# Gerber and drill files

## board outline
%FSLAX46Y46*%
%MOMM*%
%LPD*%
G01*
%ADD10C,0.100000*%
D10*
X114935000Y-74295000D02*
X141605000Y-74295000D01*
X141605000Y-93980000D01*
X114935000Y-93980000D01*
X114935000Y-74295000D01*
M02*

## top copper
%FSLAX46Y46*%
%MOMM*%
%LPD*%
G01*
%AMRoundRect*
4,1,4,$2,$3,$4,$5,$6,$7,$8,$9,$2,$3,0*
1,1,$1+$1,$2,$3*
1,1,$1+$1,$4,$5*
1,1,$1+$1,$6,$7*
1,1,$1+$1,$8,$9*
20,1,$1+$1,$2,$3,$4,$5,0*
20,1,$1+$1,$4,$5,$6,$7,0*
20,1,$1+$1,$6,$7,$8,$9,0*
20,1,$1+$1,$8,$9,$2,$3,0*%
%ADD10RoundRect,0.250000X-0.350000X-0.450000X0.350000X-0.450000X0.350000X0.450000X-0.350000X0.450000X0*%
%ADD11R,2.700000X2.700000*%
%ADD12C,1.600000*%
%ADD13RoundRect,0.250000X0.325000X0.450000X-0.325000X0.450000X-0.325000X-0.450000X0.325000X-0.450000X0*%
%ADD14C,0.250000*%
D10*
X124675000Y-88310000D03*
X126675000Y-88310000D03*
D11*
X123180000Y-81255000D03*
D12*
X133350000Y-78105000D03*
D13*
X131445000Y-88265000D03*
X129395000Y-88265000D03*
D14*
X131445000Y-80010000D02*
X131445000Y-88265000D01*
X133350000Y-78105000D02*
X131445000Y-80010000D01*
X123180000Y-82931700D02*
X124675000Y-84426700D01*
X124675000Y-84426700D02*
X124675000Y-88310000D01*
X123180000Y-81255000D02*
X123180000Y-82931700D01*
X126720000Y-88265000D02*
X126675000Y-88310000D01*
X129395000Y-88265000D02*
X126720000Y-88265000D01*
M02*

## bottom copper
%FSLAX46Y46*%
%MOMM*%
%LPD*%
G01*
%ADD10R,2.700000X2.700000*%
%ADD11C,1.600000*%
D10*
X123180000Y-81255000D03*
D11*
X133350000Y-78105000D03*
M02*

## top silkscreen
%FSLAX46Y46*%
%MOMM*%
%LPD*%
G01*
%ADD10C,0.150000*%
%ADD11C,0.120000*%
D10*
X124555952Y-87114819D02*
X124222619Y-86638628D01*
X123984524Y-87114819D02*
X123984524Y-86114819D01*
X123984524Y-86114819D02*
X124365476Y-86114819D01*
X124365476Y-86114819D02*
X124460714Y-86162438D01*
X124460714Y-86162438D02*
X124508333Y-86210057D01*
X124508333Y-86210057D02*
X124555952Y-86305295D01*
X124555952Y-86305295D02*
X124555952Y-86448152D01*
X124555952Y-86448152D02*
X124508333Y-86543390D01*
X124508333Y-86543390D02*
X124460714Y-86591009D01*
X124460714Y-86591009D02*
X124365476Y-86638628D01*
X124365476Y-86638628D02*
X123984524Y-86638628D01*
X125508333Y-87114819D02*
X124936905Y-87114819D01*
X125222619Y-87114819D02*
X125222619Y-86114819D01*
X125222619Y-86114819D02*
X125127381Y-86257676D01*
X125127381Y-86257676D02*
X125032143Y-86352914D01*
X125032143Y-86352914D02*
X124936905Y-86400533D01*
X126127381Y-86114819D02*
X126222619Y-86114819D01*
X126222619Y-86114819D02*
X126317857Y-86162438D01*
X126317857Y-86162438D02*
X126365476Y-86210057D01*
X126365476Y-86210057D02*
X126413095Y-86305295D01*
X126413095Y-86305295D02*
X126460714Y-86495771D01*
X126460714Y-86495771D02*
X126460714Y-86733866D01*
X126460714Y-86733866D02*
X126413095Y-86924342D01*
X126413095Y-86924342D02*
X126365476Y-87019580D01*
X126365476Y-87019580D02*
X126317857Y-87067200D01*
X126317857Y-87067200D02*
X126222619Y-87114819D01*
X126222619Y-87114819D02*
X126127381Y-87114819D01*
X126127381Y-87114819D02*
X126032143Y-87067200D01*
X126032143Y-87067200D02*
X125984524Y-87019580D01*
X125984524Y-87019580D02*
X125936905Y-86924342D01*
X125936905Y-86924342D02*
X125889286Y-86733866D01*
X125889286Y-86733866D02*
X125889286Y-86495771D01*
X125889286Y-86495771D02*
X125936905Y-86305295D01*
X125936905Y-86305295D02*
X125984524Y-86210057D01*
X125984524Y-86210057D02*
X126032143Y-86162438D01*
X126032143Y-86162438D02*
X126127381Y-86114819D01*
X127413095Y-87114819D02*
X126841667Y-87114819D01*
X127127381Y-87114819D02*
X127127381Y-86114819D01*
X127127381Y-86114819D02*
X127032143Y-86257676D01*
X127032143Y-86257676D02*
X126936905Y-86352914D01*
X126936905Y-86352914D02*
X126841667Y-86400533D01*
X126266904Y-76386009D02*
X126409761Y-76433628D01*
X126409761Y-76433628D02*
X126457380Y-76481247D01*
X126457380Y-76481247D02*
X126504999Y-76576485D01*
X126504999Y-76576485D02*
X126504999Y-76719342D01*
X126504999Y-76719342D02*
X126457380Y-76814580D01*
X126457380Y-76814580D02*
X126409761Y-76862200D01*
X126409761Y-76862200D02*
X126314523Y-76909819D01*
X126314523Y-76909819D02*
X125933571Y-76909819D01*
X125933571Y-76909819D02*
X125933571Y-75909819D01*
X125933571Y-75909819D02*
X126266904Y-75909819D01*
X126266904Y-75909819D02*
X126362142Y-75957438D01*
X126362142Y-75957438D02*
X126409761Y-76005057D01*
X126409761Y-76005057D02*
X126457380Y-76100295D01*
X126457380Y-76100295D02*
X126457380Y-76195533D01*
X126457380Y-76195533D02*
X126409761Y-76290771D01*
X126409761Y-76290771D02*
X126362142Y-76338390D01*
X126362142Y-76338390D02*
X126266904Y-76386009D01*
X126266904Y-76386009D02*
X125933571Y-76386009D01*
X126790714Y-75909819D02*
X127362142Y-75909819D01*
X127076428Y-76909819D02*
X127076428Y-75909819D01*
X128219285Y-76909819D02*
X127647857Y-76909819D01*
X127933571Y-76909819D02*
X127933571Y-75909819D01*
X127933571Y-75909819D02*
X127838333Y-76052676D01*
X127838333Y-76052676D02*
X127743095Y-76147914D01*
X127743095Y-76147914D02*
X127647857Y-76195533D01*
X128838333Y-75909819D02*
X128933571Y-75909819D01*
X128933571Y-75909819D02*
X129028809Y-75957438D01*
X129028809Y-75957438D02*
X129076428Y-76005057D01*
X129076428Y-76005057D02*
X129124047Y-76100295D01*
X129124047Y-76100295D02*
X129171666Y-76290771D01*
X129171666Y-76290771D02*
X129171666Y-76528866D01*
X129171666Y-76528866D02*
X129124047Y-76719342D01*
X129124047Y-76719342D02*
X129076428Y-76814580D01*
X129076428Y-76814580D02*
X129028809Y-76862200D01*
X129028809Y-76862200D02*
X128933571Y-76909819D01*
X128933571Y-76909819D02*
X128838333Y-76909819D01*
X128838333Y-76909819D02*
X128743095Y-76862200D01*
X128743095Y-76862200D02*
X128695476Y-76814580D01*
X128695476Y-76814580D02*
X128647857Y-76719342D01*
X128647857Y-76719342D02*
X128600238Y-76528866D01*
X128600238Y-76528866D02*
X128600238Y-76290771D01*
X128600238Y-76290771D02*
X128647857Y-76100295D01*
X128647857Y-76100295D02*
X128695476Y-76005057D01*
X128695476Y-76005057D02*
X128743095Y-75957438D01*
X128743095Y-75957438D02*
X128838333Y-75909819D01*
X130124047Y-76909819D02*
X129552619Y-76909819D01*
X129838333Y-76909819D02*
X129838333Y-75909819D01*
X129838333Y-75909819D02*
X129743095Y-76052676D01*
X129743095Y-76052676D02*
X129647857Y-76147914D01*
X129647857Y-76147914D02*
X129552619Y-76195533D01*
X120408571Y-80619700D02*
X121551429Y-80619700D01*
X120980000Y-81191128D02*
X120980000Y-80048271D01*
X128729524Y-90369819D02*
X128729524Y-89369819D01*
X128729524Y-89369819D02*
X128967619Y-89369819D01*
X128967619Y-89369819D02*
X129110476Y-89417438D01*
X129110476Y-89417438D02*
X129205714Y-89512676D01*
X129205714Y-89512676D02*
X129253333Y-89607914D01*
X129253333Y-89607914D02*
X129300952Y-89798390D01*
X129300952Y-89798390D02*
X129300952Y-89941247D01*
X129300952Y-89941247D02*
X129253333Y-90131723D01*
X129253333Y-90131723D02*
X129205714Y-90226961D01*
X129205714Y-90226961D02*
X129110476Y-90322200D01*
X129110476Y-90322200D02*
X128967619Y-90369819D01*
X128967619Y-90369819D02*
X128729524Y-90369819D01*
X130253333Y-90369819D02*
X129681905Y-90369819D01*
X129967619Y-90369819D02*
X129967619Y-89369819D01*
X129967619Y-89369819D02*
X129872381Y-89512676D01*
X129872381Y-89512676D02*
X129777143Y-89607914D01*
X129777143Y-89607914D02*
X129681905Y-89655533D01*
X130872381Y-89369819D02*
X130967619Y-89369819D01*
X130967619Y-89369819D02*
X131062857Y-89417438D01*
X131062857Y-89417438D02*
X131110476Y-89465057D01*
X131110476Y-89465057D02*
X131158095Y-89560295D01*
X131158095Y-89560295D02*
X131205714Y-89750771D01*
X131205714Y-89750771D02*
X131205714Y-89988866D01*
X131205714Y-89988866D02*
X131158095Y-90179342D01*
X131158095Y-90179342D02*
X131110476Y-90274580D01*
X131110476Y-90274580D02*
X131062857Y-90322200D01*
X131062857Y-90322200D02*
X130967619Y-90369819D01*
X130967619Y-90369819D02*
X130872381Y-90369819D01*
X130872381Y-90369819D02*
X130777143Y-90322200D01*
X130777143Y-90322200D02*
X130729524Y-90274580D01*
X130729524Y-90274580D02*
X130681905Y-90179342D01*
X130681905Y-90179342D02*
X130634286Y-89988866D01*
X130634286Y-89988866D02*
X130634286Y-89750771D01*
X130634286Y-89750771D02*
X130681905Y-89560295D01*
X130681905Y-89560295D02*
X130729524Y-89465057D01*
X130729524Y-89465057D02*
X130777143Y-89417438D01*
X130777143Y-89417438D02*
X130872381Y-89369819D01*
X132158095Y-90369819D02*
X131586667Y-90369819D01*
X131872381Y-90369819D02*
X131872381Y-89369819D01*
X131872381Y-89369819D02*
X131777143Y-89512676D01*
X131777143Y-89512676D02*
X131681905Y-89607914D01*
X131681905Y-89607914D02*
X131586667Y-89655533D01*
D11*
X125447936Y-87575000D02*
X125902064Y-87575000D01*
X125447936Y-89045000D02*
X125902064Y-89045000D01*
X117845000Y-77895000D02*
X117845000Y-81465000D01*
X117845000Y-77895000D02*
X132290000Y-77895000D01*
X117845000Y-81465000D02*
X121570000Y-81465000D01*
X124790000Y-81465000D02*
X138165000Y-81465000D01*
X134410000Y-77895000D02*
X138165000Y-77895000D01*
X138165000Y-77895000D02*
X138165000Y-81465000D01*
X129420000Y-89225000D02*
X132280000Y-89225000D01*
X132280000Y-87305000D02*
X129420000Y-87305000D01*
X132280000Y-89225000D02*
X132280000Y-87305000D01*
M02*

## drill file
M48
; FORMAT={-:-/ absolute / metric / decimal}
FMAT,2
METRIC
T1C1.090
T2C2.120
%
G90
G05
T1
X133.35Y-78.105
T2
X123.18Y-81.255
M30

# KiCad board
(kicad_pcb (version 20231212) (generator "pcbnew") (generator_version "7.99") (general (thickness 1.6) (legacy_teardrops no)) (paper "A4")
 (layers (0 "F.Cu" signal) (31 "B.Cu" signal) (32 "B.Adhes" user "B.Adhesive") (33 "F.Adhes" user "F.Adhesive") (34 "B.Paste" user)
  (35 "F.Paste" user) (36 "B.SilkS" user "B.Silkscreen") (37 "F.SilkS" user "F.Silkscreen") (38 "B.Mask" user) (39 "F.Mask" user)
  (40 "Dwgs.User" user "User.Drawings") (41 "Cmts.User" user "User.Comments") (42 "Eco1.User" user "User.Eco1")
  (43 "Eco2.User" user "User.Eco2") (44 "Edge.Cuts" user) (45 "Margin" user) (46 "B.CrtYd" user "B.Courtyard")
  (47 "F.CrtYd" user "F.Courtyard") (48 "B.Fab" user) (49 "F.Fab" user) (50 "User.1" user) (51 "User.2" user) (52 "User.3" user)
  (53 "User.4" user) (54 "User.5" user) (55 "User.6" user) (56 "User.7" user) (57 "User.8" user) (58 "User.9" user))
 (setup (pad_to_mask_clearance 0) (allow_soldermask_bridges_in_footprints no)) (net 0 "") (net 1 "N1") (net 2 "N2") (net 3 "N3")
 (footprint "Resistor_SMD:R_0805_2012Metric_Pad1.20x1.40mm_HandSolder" (layer "F.Cu") (at 125.675 88.31)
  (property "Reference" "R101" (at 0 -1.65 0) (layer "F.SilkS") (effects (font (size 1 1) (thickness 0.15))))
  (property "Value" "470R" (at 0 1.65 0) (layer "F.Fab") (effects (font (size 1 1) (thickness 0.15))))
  (fp_line (start -0.227064 -0.735) (end 0.227064 -0.735) (stroke (width 0.12) (type solid)) (layer "F.SilkS"))
  (fp_line (start -0.227064 0.735) (end 0.227064 0.735) (stroke (width 0.12) (type solid)) (layer "F.SilkS"))
  (pad "1" smd roundrect (at -1 0) (size 1.2 1.4) (layers "F.Cu" "F.Paste" "F.Mask") (roundrect_rratio 0.208333) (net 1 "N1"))
  (pad "2" smd roundrect (at 1 0) (size 1.2 1.4) (layers "F.Cu" "F.Paste" "F.Mask") (roundrect_rratio 0.208333) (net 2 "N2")))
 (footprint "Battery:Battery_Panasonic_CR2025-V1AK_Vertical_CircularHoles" (layer "F.Cu") (at 123.18 81.255)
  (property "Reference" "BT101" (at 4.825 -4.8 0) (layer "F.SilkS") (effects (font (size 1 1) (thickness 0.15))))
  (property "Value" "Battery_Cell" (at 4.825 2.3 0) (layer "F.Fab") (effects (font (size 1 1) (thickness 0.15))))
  (fp_line (start -5.335 -3.36) (end -5.335 0.21) (stroke (width 0.12) (type solid)) (layer "F.SilkS"))
  (fp_line (start -5.335 -3.36) (end 9.11 -3.36) (stroke (width 0.12) (type solid)) (layer "F.SilkS"))
  (fp_line (start -5.335 0.21) (end -1.61 0.21) (stroke (width 0.12) (type solid)) (layer "F.SilkS"))
  (fp_line (start 1.61 0.21) (end 14.985 0.21) (stroke (width 0.12) (type solid)) (layer "F.SilkS"))
  (fp_line (start 11.23 -3.36) (end 14.985 -3.36) (stroke (width 0.12) (type solid)) (layer "F.SilkS"))
  (fp_line (start 14.985 -3.36) (end 14.985 0.21) (stroke (width 0.12) (type solid)) (layer "F.SilkS"))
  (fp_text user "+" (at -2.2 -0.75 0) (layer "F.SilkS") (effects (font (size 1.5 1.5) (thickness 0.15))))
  (pad "1" thru_hole rect (at 0 0 90) (size 2.7 2.7) (drill 2.12) (layers "*.Cu" "*.Mask") (remove_unused_layers no) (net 1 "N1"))
  (pad "2" thru_hole circle (at 10.17 -3.15) (size 1.6 1.6) (drill 1.09) (layers "*.Cu" "*.Mask") (remove_unused_layers no) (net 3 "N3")))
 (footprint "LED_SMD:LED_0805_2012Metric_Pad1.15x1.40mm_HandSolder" (layer "F.Cu") (at 130.42 88.265 180)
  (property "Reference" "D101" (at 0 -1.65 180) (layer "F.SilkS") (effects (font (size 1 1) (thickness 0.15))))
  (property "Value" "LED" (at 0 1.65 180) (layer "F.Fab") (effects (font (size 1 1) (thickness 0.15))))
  (fp_line (start 1 -0.96) (end -1.86 -0.96) (stroke (width 0.12) (type solid)) (layer "F.SilkS"))
  (fp_line (start -1.86 0.96) (end 1 0.96) (stroke (width 0.12) (type solid)) (layer "F.SilkS"))
  (fp_line (start -1.86 -0.96) (end -1.86 0.96) (stroke (width 0.12) (type solid)) (layer "F.SilkS"))
  (pad "1" smd roundrect (at -1.025 0 180) (size 1.15 1.4) (layers "F.Cu" "F.Paste" "F.Mask") (roundrect_rratio 0.217391) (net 3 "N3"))
  (pad "2" smd roundrect (at 1.025 0 180) (size 1.15 1.4) (layers "F.Cu" "F.Paste" "F.Mask") (roundrect_rratio 0.217391) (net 2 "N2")))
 (gr_rect (start 114.935 74.295) (end 141.605 93.98) (stroke (width 0.1) (type default)) (fill none) (layer "Edge.Cuts"))
 (segment (start 131.445 80.01) (end 131.445 88.265) (width 0.25) (layer "F.Cu") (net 3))
 (segment (start 133.35 78.105) (end 131.445 80.01) (width 0.25) (layer "F.Cu") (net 3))
 (segment (start 123.18 82.9317) (end 124.675 84.4267) (width 0.25) (layer "F.Cu") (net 1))
 (segment (start 124.675 84.4267) (end 124.675 88.31) (width 0.25) (layer "F.Cu") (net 1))
 (segment (start 123.18 81.255) (end 123.18 82.9317) (width 0.25) (layer "F.Cu") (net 1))
 (segment (start 126.72 88.265) (end 126.675 88.31) (width 0.25) (layer "F.Cu") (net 2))
 (segment (start 129.395 88.265) (end 126.72 88.265) (width 0.25) (layer "F.Cu") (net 2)))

